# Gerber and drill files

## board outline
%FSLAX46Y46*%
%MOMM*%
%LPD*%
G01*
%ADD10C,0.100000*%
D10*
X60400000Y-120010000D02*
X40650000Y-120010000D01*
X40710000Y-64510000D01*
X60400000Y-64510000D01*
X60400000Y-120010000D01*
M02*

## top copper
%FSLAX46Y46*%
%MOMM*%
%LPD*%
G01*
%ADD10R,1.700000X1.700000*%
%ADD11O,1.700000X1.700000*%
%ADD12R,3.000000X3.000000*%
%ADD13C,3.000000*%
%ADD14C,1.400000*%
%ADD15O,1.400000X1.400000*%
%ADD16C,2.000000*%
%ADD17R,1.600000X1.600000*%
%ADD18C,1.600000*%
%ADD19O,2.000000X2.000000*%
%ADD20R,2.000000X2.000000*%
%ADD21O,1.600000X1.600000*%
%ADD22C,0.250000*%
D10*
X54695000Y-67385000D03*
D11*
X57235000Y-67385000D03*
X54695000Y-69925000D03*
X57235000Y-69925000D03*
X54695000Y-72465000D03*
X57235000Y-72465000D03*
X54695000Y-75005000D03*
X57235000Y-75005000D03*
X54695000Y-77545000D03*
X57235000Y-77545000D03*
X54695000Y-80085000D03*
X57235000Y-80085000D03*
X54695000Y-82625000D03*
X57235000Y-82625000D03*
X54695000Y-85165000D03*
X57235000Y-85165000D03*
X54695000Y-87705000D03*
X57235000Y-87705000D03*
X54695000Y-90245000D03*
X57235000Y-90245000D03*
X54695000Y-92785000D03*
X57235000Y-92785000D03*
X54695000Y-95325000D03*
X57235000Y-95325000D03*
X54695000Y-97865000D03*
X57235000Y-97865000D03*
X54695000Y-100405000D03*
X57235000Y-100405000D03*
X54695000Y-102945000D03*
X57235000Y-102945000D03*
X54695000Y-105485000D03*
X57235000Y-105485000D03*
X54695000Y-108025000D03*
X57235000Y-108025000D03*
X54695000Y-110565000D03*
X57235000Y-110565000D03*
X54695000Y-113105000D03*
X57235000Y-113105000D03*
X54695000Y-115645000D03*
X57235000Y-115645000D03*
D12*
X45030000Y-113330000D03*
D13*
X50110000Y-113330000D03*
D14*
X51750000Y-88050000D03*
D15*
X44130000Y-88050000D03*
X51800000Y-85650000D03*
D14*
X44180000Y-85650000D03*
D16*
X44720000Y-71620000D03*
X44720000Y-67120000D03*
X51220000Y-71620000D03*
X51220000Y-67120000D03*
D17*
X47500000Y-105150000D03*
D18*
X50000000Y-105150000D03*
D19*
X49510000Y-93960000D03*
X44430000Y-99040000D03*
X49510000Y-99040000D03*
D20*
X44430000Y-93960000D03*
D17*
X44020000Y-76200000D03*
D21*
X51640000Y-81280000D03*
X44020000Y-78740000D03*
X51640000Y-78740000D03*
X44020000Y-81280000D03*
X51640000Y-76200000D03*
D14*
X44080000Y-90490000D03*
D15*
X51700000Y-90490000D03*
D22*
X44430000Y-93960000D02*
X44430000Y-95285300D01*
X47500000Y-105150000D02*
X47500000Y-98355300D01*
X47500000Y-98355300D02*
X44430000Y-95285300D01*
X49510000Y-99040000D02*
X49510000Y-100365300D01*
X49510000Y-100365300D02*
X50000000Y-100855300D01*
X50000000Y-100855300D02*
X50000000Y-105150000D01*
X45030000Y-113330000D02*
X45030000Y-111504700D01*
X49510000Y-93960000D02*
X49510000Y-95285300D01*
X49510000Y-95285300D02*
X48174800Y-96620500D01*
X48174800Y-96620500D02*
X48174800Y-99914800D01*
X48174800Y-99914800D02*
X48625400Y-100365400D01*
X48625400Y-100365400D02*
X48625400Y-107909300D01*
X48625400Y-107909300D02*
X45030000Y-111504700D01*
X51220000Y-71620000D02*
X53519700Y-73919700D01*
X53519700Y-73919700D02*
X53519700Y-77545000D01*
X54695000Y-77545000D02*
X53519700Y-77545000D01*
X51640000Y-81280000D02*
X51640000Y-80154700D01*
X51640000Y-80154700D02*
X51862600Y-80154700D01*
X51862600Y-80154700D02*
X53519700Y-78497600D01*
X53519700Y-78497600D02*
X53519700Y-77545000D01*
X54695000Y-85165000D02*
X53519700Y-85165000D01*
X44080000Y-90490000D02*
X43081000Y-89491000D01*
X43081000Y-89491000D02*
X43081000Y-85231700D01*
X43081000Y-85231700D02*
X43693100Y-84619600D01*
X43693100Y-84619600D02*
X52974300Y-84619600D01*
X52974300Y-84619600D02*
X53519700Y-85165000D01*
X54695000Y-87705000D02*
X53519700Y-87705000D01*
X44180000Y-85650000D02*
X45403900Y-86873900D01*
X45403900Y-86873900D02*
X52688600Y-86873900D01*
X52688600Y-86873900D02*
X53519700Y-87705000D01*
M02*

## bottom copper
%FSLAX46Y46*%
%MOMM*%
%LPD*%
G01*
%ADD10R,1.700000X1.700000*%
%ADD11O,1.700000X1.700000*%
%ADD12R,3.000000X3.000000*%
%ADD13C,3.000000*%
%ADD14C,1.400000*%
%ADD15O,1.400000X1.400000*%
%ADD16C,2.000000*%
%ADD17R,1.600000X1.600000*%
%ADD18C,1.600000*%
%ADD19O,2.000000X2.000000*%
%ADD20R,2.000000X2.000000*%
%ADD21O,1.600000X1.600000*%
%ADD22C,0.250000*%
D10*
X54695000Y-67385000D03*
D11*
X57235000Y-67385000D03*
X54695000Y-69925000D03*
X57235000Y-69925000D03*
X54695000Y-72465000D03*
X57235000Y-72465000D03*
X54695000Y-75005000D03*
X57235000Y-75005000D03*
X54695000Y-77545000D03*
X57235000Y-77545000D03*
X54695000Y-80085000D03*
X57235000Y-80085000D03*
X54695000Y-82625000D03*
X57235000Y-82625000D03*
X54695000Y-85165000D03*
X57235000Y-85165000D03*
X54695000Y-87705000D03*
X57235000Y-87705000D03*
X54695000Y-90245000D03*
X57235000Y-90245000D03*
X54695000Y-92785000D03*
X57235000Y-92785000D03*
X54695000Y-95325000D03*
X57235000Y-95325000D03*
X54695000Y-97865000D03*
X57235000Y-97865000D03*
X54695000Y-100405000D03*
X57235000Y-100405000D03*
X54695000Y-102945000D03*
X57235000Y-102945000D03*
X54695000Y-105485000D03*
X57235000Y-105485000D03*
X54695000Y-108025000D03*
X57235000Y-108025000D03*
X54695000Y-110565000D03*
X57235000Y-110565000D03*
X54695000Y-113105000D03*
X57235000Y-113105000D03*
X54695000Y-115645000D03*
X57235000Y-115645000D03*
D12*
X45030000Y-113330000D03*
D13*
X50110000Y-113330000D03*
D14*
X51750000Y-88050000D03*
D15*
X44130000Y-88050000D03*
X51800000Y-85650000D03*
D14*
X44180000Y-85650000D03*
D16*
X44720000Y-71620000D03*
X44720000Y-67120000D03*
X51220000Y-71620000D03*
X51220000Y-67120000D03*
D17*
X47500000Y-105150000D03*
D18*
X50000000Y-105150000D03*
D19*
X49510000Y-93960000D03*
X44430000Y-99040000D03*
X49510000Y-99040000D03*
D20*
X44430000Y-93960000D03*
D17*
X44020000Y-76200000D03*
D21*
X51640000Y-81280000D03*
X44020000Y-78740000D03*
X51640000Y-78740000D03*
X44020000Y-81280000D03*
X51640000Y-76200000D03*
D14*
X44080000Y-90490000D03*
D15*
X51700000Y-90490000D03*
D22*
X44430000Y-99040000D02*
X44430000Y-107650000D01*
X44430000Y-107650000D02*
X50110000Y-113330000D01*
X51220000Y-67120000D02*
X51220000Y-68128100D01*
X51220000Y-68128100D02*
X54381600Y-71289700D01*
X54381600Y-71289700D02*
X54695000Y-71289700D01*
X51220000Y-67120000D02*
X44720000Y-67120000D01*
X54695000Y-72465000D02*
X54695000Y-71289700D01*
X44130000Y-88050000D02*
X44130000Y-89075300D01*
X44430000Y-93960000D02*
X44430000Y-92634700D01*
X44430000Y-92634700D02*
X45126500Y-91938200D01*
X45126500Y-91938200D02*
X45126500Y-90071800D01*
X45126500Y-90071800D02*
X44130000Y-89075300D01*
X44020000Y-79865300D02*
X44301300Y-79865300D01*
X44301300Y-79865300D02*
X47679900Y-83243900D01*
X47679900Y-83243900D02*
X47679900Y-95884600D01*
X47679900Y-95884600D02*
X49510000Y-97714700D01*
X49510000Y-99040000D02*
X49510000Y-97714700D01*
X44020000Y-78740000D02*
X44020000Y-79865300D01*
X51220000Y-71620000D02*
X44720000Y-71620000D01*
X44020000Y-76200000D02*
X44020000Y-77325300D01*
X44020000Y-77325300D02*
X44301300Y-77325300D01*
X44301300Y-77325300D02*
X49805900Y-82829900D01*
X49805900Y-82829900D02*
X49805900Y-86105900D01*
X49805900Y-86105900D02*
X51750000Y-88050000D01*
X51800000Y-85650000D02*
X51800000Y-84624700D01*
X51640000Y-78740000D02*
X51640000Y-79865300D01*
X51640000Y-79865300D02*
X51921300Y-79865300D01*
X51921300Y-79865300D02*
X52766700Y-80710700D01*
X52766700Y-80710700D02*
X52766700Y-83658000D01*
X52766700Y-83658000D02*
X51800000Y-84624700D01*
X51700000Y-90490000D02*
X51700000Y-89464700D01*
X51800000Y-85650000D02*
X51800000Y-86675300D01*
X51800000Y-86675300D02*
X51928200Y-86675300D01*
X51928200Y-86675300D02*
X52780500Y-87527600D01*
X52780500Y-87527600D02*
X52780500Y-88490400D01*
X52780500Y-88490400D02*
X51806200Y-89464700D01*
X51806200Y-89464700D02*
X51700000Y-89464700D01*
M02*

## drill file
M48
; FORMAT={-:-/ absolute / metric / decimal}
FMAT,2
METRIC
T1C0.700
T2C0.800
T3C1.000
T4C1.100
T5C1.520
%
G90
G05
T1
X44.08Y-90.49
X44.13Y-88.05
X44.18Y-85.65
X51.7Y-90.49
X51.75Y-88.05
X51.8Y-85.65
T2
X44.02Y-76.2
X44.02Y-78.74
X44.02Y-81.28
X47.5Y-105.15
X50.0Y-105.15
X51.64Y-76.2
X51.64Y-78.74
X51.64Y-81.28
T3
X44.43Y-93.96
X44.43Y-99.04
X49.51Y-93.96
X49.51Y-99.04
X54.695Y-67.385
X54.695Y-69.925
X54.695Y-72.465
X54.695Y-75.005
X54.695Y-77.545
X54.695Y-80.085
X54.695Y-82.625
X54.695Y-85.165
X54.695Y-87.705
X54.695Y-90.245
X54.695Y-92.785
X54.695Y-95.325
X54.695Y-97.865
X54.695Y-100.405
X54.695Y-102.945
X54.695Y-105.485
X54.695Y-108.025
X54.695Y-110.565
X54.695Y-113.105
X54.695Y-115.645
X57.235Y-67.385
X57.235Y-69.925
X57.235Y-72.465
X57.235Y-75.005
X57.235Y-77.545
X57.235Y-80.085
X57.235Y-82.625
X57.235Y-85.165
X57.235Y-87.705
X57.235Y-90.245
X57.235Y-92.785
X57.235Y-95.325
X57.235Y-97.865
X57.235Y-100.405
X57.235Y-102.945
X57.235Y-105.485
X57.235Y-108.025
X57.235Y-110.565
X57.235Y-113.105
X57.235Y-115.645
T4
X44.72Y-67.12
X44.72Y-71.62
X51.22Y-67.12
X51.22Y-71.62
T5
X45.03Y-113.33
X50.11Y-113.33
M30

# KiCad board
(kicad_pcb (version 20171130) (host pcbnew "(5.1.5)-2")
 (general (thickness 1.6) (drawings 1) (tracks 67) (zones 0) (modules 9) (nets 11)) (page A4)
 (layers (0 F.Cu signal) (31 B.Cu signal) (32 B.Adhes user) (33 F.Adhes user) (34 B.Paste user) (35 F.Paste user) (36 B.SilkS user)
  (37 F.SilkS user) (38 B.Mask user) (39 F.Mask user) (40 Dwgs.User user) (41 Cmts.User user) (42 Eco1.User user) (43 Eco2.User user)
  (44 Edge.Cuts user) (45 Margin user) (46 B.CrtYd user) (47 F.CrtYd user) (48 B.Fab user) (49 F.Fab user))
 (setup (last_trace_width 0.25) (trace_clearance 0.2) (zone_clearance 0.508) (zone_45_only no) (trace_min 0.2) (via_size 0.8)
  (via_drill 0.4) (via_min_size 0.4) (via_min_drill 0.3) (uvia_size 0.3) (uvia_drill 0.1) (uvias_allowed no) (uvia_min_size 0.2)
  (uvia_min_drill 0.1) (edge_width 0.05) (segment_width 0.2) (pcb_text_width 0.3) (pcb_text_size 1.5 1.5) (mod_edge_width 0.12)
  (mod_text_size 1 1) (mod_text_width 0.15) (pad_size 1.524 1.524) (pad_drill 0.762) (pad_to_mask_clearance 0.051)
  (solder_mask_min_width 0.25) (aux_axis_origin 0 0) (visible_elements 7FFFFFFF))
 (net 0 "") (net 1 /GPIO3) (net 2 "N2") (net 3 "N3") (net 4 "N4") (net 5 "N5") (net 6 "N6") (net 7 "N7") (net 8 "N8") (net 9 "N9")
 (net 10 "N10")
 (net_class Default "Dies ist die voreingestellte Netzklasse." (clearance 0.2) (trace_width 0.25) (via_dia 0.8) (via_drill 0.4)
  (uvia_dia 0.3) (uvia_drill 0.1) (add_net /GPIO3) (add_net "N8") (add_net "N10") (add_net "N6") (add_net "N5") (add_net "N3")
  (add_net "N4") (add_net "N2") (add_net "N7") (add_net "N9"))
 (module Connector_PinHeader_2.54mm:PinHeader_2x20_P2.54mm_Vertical (layer F.Cu) (at 54.695 67.385)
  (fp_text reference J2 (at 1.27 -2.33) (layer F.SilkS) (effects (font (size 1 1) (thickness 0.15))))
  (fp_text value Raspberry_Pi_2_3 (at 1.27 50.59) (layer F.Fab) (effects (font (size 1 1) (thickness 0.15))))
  (pad 1 thru_hole rect (at 0 0) (size 1.7 1.7) (drill 1) (layers *.Cu *.Mask))
  (pad 2 thru_hole oval (at 2.54 0) (size 1.7 1.7) (drill 1) (layers *.Cu *.Mask))
  (pad 3 thru_hole oval (at 0 2.54) (size 1.7 1.7) (drill 1) (layers *.Cu *.Mask))
  (pad 4 thru_hole oval (at 2.54 2.54) (size 1.7 1.7) (drill 1) (layers *.Cu *.Mask))
  (pad 5 thru_hole oval (at 0 5.08) (size 1.7 1.7) (drill 1) (layers *.Cu *.Mask) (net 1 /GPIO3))
  (pad 6 thru_hole oval (at 2.54 5.08) (size 1.7 1.7) (drill 1) (layers *.Cu *.Mask))
  (pad 7 thru_hole oval (at 0 7.62) (size 1.7 1.7) (drill 1) (layers *.Cu *.Mask))
  (pad 8 thru_hole oval (at 2.54 7.62) (size 1.7 1.7) (drill 1) (layers *.Cu *.Mask))
  (pad 9 thru_hole oval (at 0 10.16) (size 1.7 1.7) (drill 1) (layers *.Cu *.Mask) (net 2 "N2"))
  (pad 10 thru_hole oval (at 2.54 10.16) (size 1.7 1.7) (drill 1) (layers *.Cu *.Mask))
  (pad 11 thru_hole oval (at 0 12.7) (size 1.7 1.7) (drill 1) (layers *.Cu *.Mask))
  (pad 12 thru_hole oval (at 2.54 12.7) (size 1.7 1.7) (drill 1) (layers *.Cu *.Mask))
  (pad 13 thru_hole oval (at 0 15.24) (size 1.7 1.7) (drill 1) (layers *.Cu *.Mask))
  (pad 14 thru_hole oval (at 2.54 15.24) (size 1.7 1.7) (drill 1) (layers *.Cu *.Mask))
  (pad 15 thru_hole oval (at 0 17.78) (size 1.7 1.7) (drill 1) (layers *.Cu *.Mask) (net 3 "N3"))
  (pad 16 thru_hole oval (at 2.54 17.78) (size 1.7 1.7) (drill 1) (layers *.Cu *.Mask))
  (pad 17 thru_hole oval (at 0 20.32) (size 1.7 1.7) (drill 1) (layers *.Cu *.Mask) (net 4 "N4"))
  (pad 18 thru_hole oval (at 2.54 20.32) (size 1.7 1.7) (drill 1) (layers *.Cu *.Mask))
  (pad 19 thru_hole oval (at 0 22.86) (size 1.7 1.7) (drill 1) (layers *.Cu *.Mask))
  (pad 20 thru_hole oval (at 2.54 22.86) (size 1.7 1.7) (drill 1) (layers *.Cu *.Mask))
  (pad 21 thru_hole oval (at 0 25.4) (size 1.7 1.7) (drill 1) (layers *.Cu *.Mask))
  (pad 22 thru_hole oval (at 2.54 25.4) (size 1.7 1.7) (drill 1) (layers *.Cu *.Mask))
  (pad 23 thru_hole oval (at 0 27.94) (size 1.7 1.7) (drill 1) (layers *.Cu *.Mask))
  (pad 24 thru_hole oval (at 2.54 27.94) (size 1.7 1.7) (drill 1) (layers *.Cu *.Mask))
  (pad 25 thru_hole oval (at 0 30.48) (size 1.7 1.7) (drill 1) (layers *.Cu *.Mask))
  (pad 26 thru_hole oval (at 2.54 30.48) (size 1.7 1.7) (drill 1) (layers *.Cu *.Mask))
  (pad 27 thru_hole oval (at 0 33.02) (size 1.7 1.7) (drill 1) (layers *.Cu *.Mask))
  (pad 28 thru_hole oval (at 2.54 33.02) (size 1.7 1.7) (drill 1) (layers *.Cu *.Mask))
  (pad 29 thru_hole oval (at 0 35.56) (size 1.7 1.7) (drill 1) (layers *.Cu *.Mask))
  (pad 30 thru_hole oval (at 2.54 35.56) (size 1.7 1.7) (drill 1) (layers *.Cu *.Mask))
  (pad 31 thru_hole oval (at 0 38.1) (size 1.7 1.7) (drill 1) (layers *.Cu *.Mask))
  (pad 32 thru_hole oval (at 2.54 38.1) (size 1.7 1.7) (drill 1) (layers *.Cu *.Mask))
  (pad 33 thru_hole oval (at 0 40.64) (size 1.7 1.7) (drill 1) (layers *.Cu *.Mask))
  (pad 34 thru_hole oval (at 2.54 40.64) (size 1.7 1.7) (drill 1) (layers *.Cu *.Mask))
  (pad 35 thru_hole oval (at 0 43.18) (size 1.7 1.7) (drill 1) (layers *.Cu *.Mask))
  (pad 36 thru_hole oval (at 2.54 43.18) (size 1.7 1.7) (drill 1) (layers *.Cu *.Mask))
  (pad 37 thru_hole oval (at 0 45.72) (size 1.7 1.7) (drill 1) (layers *.Cu *.Mask))
  (pad 38 thru_hole oval (at 2.54 45.72) (size 1.7 1.7) (drill 1) (layers *.Cu *.Mask))
  (pad 39 thru_hole oval (at 0 48.26) (size 1.7 1.7) (drill 1) (layers *.Cu *.Mask))
  (pad 40 thru_hole oval (at 2.54 48.26) (size 1.7 1.7) (drill 1) (layers *.Cu *.Mask)))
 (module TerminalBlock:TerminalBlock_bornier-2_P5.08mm (layer F.Cu) (at 45.03 113.33)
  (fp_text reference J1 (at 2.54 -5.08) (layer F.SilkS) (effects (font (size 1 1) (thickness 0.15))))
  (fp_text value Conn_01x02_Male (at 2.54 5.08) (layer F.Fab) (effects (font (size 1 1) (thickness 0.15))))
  (pad 1 thru_hole rect (at 0 0) (size 3 3) (drill 1.52) (layers *.Cu *.Mask) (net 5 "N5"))
  (pad 2 thru_hole circle (at 5.08 0) (size 3 3) (drill 1.52) (layers *.Cu *.Mask) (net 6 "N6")))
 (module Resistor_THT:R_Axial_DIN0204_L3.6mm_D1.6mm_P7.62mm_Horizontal (layer F.Cu) (at 51.75 88.05 180)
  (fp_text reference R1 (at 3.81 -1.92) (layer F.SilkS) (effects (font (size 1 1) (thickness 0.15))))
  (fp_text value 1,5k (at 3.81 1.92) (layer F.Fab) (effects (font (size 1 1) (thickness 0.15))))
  (pad 1 thru_hole circle (at 0 0 180) (size 1.4 1.4) (drill 0.7) (layers *.Cu *.Mask) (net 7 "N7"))
  (pad 2 thru_hole oval (at 7.62 0 180) (size 1.4 1.4) (drill 0.7) (layers *.Cu *.Mask) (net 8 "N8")))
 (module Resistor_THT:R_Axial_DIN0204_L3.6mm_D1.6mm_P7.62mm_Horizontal (layer F.Cu) (at 44.18 85.65)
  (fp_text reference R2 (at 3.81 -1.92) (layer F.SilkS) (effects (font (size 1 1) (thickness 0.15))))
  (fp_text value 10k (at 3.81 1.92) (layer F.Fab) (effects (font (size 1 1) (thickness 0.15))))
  (pad 2 thru_hole oval (at 7.62 0) (size 1.4 1.4) (drill 0.7) (layers *.Cu *.Mask) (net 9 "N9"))
  (pad 1 thru_hole circle (at 0 0) (size 1.4 1.4) (drill 0.7) (layers *.Cu *.Mask) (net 4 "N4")))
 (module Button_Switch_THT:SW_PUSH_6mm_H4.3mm (layer F.Cu) (at 44.72 67.12)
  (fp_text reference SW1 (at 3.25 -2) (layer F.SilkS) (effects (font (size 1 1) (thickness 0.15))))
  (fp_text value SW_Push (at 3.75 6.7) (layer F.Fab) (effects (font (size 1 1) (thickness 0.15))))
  (pad 2 thru_hole circle (at 0 4.5 90) (size 2 2) (drill 1.1) (layers *.Cu *.Mask) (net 2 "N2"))
  (pad 1 thru_hole circle (at 0 0 90) (size 2 2) (drill 1.1) (layers *.Cu *.Mask) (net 1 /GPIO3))
  (pad 2 thru_hole circle (at 6.5 4.5 90) (size 2 2) (drill 1.1) (layers *.Cu *.Mask) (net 2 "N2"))
  (pad 1 thru_hole circle (at 6.5 0 90) (size 2 2) (drill 1.1) (layers *.Cu *.Mask) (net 1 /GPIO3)))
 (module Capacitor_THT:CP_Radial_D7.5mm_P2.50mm (layer F.Cu) (at 47.5 105.15)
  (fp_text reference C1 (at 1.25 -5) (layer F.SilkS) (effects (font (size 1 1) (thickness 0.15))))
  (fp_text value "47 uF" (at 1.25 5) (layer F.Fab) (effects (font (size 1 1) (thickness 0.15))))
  (pad 1 thru_hole rect (at 0 0) (size 1.6 1.6) (drill 0.8) (layers *.Cu *.Mask) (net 8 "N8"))
  (pad 2 thru_hole circle (at 2.5 0) (size 1.6 1.6) (drill 0.8) (layers *.Cu *.Mask) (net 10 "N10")))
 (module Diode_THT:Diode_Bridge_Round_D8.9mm (layer F.Cu) (at 44.43 93.96)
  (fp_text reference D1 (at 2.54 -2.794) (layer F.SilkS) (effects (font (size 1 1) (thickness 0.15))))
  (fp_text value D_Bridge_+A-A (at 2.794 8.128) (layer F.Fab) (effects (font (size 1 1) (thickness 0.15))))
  (pad 4 thru_hole oval (at 5.08 0) (size 2 2) (drill 1) (layers *.Cu *.Mask) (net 5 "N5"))
  (pad 2 thru_hole oval (at 0 5.08) (size 2 2) (drill 1) (layers *.Cu *.Mask) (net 6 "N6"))
  (pad 3 thru_hole oval (at 5.08 5.08) (size 2 2) (drill 1) (layers *.Cu *.Mask) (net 10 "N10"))
  (pad 1 thru_hole rect (at 0 0) (size 2 2) (drill 1) (layers *.Cu *.Mask) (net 8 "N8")))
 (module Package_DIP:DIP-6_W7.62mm (layer F.Cu) (at 44.02 76.2)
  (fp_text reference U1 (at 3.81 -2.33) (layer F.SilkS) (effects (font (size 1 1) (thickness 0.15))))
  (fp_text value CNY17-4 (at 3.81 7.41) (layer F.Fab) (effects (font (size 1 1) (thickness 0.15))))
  (pad 1 thru_hole rect (at 0 0) (size 1.6 1.6) (drill 0.8) (layers *.Cu *.Mask) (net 7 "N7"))
  (pad 4 thru_hole oval (at 7.62 5.08) (size 1.6 1.6) (drill 0.8) (layers *.Cu *.Mask) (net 2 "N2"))
  (pad 2 thru_hole oval (at 0 2.54) (size 1.6 1.6) (drill 0.8) (layers *.Cu *.Mask) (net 10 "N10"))
  (pad 5 thru_hole oval (at 7.62 2.54) (size 1.6 1.6) (drill 0.8) (layers *.Cu *.Mask) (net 9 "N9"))
  (pad 3 thru_hole oval (at 0 5.08) (size 1.6 1.6) (drill 0.8) (layers *.Cu *.Mask))
  (pad 6 thru_hole oval (at 7.62 0) (size 1.6 1.6) (drill 0.8) (layers *.Cu *.Mask)))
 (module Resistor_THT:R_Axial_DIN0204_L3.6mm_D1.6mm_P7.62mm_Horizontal (layer F.Cu) (at 44.08 90.49)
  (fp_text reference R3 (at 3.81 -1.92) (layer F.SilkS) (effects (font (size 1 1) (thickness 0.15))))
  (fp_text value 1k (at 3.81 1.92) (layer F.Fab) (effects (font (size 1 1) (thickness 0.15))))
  (pad 1 thru_hole circle (at 0 0) (size 1.4 1.4) (drill 0.7) (layers *.Cu *.Mask) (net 3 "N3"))
  (pad 2 thru_hole oval (at 7.62 0) (size 1.4 1.4) (drill 0.7) (layers *.Cu *.Mask) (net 9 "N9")))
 (gr_poly (pts (xy 60.4 120.01) (xy 40.65 120.01) (xy 40.71 64.51) (xy 60.4 64.51)) (layer Edge.Cuts) (width 0.1))
 (segment (start 44.43 99.04) (end 44.43 107.65) (width 0.25) (layer B.Cu) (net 6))
 (segment (start 44.43 107.65) (end 50.11 113.33) (width 0.25) (layer B.Cu) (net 6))
 (segment (start 51.22 67.12) (end 51.22 68.1281) (width 0.25) (layer B.Cu) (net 1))
 (segment (start 51.22 68.1281) (end 54.3816 71.2897) (width 0.25) (layer B.Cu) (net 1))
 (segment (start 54.3816 71.2897) (end 54.695 71.2897) (width 0.25) (layer B.Cu) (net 1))
 (segment (start 51.22 67.12) (end 44.72 67.12) (width 0.25) (layer B.Cu) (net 1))
 (segment (start 54.695 72.465) (end 54.695 71.2897) (width 0.25) (layer B.Cu) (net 1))
 (segment (start 44.13 88.05) (end 44.13 89.0753) (width 0.25) (layer B.Cu) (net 8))
 (segment (start 44.43 93.96) (end 44.43 92.6347) (width 0.25) (layer B.Cu) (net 8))
 (segment (start 44.43 92.6347) (end 45.1265 91.9382) (width 0.25) (layer B.Cu) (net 8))
 (segment (start 45.1265 91.9382) (end 45.1265 90.0718) (width 0.25) (layer B.Cu) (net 8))
 (segment (start 45.1265 90.0718) (end 44.13 89.0753) (width 0.25) (layer B.Cu) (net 8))
 (segment (start 44.43 93.96) (end 44.43 95.2853) (width 0.25) (layer F.Cu) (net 8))
 (segment (start 47.5 105.15) (end 47.5 98.3553) (width 0.25) (layer F.Cu) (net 8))
 (segment (start 47.5 98.3553) (end 44.43 95.2853) (width 0.25) (layer F.Cu) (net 8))
 (segment (start 44.02 79.8653) (end 44.3013 79.8653) (width 0.25) (layer B.Cu) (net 10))
 (segment (start 44.3013 79.8653) (end 47.6799 83.2439) (width 0.25) (layer B.Cu) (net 10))
 (segment (start 47.6799 83.2439) (end 47.6799 95.8846) (width 0.25) (layer B.Cu) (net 10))
 (segment (start 47.6799 95.8846) (end 49.51 97.7147) (width 0.25) (layer B.Cu) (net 10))
 (segment (start 49.51 99.04) (end 49.51 100.3653) (width 0.25) (layer F.Cu) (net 10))
 (segment (start 49.51 100.3653) (end 50 100.8553) (width 0.25) (layer F.Cu) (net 10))
 (segment (start 50 100.8553) (end 50 105.15) (width 0.25) (layer F.Cu) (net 10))
 (segment (start 49.51 99.04) (end 49.51 97.7147) (width 0.25) (layer B.Cu) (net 10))
 (segment (start 44.02 78.74) (end 44.02 79.8653) (width 0.25) (layer B.Cu) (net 10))
 (segment (start 45.03 113.33) (end 45.03 111.5047) (width 0.25) (layer F.Cu) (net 5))
 (segment (start 49.51 93.96) (end 49.51 95.2853) (width 0.25) (layer F.Cu) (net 5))
 (segment (start 49.51 95.2853) (end 48.1748 96.6205) (width 0.25) (layer F.Cu) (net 5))
 (segment (start 48.1748 96.6205) (end 48.1748 99.9148) (width 0.25) (layer F.Cu) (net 5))
 (segment (start 48.1748 99.9148) (end 48.6254 100.3654) (width 0.25) (layer F.Cu) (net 5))
 (segment (start 48.6254 100.3654) (end 48.6254 107.9093) (width 0.25) (layer F.Cu) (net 5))
 (segment (start 48.6254 107.9093) (end 45.03 111.5047) (width 0.25) (layer F.Cu) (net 5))
 (segment (start 51.22 71.62) (end 53.5197 73.9197) (width 0.25) (layer F.Cu) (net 2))
 (segment (start 53.5197 73.9197) (end 53.5197 77.545) (width 0.25) (layer F.Cu) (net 2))
 (segment (start 54.695 77.545) (end 53.5197 77.545) (width 0.25) (layer F.Cu) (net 2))
 (segment (start 51.64 81.28) (end 51.64 80.1547) (width 0.25) (layer F.Cu) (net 2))
 (segment (start 51.64 80.1547) (end 51.8626 80.1547) (width 0.25) (layer F.Cu) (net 2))
 (segment (start 51.8626 80.1547) (end 53.5197 78.4976) (width 0.25) (layer F.Cu) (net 2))
 (segment (start 53.5197 78.4976) (end 53.5197 77.545) (width 0.25) (layer F.Cu) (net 2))
 (segment (start 51.22 71.62) (end 44.72 71.62) (width 0.25) (layer B.Cu) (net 2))
 (segment (start 54.695 85.165) (end 53.5197 85.165) (width 0.25) (layer F.Cu) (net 3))
 (segment (start 44.08 90.49) (end 43.081 89.491) (width 0.25) (layer F.Cu) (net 3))
 (segment (start 43.081 89.491) (end 43.081 85.2317) (width 0.25) (layer F.Cu) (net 3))
 (segment (start 43.081 85.2317) (end 43.6931 84.6196) (width 0.25) (layer F.Cu) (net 3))
 (segment (start 43.6931 84.6196) (end 52.9743 84.6196) (width 0.25) (layer F.Cu) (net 3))
 (segment (start 52.9743 84.6196) (end 53.5197 85.165) (width 0.25) (layer F.Cu) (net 3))
 (segment (start 54.695 87.705) (end 53.5197 87.705) (width 0.25) (layer F.Cu) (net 4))
 (segment (start 44.18 85.65) (end 45.4039 86.8739) (width 0.25) (layer F.Cu) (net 4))
 (segment (start 45.4039 86.8739) (end 52.6886 86.8739) (width 0.25) (layer F.Cu) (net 4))
 (segment (start 52.6886 86.8739) (end 53.5197 87.705) (width 0.25) (layer F.Cu) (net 4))
 (segment (start 44.02 76.2) (end 44.02 77.3253) (width 0.25) (layer B.Cu) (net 7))
 (segment (start 44.02 77.3253) (end 44.3013 77.3253) (width 0.25) (layer B.Cu) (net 7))
 (segment (start 44.3013 77.3253) (end 49.8059 82.8299) (width 0.25) (layer B.Cu) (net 7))
 (segment (start 49.8059 82.8299) (end 49.8059 86.1059) (width 0.25) (layer B.Cu) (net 7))
 (segment (start 49.8059 86.1059) (end 51.75 88.05) (width 0.25) (layer B.Cu) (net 7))
 (segment (start 51.8 85.65) (end 51.8 84.6247) (width 0.25) (layer B.Cu) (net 9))
 (segment (start 51.64 78.74) (end 51.64 79.8653) (width 0.25) (layer B.Cu) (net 9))
 (segment (start 51.64 79.8653) (end 51.9213 79.8653) (width 0.25) (layer B.Cu) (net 9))
 (segment (start 51.9213 79.8653) (end 52.7667 80.7107) (width 0.25) (layer B.Cu) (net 9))
 (segment (start 52.7667 80.7107) (end 52.7667 83.658) (width 0.25) (layer B.Cu) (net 9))
 (segment (start 52.7667 83.658) (end 51.8 84.6247) (width 0.25) (layer B.Cu) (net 9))
 (segment (start 51.7 90.49) (end 51.7 89.4647) (width 0.25) (layer B.Cu) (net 9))
 (segment (start 51.8 85.65) (end 51.8 86.6753) (width 0.25) (layer B.Cu) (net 9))
 (segment (start 51.8 86.6753) (end 51.9282 86.6753) (width 0.25) (layer B.Cu) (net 9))
 (segment (start 51.9282 86.6753) (end 52.7805 87.5276) (width 0.25) (layer B.Cu) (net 9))
 (segment (start 52.7805 87.5276) (end 52.7805 88.4904) (width 0.25) (layer B.Cu) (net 9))
 (segment (start 52.7805 88.4904) (end 51.8062 89.4647) (width 0.25) (layer B.Cu) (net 9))
 (segment (start 51.8062 89.4647) (end 51.7 89.4647) (width 0.25) (layer B.Cu) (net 9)))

